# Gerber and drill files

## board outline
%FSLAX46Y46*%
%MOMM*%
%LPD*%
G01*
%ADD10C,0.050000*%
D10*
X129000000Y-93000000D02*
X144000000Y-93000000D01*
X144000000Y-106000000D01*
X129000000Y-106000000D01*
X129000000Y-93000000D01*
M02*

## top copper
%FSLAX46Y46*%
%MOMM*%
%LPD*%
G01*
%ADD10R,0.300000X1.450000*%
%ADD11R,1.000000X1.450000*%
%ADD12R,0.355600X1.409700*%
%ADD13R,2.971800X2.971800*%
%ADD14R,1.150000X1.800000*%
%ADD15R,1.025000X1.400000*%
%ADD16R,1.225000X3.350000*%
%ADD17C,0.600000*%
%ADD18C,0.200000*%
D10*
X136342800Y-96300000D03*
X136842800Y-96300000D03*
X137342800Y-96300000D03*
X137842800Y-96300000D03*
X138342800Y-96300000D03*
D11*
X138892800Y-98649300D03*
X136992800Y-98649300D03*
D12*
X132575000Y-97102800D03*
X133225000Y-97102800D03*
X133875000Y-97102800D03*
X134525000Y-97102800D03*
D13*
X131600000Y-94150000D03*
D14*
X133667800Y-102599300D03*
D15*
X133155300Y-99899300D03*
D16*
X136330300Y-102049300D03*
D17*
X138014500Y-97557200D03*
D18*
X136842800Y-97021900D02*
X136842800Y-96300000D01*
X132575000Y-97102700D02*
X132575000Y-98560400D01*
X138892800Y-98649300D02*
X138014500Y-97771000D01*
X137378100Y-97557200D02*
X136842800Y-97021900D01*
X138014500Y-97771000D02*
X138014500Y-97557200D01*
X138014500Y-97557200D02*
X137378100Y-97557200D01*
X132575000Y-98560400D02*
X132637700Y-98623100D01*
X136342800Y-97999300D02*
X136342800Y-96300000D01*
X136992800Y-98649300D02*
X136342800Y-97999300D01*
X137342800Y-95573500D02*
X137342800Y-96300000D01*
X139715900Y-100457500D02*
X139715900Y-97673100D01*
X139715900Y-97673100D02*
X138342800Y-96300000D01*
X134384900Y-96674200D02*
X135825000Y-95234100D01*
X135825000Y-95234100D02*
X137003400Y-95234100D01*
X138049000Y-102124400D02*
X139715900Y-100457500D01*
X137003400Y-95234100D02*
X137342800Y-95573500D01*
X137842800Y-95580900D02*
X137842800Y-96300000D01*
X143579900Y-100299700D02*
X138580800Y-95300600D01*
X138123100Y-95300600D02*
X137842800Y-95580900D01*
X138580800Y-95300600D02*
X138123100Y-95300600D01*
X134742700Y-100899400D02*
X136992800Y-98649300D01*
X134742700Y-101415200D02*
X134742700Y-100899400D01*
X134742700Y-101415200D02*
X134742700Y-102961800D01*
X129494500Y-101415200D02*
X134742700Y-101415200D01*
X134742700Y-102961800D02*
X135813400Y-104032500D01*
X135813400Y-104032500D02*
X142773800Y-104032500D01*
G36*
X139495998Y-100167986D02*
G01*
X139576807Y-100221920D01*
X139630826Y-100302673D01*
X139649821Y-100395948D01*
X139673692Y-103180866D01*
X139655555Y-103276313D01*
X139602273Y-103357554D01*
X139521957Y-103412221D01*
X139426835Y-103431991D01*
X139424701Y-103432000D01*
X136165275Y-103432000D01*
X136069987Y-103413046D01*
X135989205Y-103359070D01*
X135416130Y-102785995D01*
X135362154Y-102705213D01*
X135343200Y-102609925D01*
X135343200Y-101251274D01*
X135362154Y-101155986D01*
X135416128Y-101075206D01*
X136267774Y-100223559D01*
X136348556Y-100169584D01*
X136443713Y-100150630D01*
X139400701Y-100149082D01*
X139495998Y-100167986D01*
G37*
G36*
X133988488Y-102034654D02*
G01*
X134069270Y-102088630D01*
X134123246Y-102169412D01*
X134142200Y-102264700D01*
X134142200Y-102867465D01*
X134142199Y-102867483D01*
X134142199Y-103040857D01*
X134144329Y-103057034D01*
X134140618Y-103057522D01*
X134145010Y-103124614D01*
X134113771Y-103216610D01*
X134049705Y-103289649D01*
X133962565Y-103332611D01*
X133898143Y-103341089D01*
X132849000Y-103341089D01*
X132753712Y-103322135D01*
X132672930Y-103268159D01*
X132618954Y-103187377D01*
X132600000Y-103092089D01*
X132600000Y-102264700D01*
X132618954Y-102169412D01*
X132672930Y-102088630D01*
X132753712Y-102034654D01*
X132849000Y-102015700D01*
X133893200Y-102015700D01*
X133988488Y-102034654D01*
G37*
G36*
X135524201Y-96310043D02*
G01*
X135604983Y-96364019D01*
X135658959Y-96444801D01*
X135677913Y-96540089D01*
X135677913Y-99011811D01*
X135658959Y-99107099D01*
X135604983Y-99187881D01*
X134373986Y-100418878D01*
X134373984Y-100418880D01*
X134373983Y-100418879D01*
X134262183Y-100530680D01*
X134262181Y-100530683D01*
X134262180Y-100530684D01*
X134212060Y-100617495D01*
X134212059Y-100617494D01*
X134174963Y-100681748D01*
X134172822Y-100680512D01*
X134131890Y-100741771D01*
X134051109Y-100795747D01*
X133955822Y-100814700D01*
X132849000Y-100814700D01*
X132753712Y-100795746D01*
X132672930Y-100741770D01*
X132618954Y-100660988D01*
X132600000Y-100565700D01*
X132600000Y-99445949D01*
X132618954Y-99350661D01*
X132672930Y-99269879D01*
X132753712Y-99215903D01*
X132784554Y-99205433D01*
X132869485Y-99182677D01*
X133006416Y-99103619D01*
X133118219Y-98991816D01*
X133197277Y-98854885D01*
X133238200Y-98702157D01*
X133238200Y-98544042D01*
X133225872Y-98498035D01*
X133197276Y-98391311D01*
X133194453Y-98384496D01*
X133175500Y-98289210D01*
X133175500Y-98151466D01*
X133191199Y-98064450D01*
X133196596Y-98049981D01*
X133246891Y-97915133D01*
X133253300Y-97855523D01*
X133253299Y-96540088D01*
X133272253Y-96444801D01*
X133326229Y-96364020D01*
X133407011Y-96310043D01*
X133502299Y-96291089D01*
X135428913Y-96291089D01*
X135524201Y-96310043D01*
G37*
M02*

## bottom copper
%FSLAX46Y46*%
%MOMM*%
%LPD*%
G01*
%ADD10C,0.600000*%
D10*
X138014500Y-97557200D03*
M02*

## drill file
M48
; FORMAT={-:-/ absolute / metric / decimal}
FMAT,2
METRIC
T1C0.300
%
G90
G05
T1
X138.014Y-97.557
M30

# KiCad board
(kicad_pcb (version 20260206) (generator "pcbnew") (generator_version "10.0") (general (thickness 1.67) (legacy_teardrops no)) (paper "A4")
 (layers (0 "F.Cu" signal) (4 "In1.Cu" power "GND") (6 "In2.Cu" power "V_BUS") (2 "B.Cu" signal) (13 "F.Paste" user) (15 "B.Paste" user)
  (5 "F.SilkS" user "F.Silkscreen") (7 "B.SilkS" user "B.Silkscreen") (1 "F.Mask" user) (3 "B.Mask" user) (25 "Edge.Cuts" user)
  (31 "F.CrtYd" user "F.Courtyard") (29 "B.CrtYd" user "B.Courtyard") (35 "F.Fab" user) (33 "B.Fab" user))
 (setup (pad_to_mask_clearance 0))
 (gr_rect (start 129 93) (end 144 106) (stroke (width 0.05) (type default)) (fill no) (layer "Edge.Cuts"))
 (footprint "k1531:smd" (layer "F.Cu") (at 136.3428 96.3) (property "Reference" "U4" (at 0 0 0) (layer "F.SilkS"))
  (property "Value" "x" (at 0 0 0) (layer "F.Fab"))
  (pad "1" smd rect (at 0 0) (size 0.3 1.45) (layers "F.Cu" "F.Mask") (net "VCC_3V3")))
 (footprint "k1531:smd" (layer "F.Cu") (at 136.8428 96.3) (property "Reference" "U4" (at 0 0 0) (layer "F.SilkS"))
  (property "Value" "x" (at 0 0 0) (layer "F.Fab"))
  (pad "1" smd rect (at 0 0) (size 0.3 1.45) (layers "F.Cu" "F.Mask") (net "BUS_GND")))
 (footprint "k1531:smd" (layer "F.Cu") (at 137.3428 96.3) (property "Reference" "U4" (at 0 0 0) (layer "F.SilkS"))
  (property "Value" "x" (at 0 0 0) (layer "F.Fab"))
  (pad "1" smd rect (at 0 0) (size 0.3 1.45) (layers "F.Cu" "F.Mask") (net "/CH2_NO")))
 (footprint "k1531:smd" (layer "F.Cu") (at 137.8428 96.3) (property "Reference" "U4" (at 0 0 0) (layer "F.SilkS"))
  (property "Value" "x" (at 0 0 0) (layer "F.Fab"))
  (pad "1" smd rect (at 0 0) (size 0.3 1.45) (layers "F.Cu" "F.Mask") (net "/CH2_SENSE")))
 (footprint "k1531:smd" (layer "F.Cu") (at 138.3428 96.3) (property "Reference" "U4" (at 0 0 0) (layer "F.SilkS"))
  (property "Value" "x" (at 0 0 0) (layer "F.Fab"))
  (pad "1" smd rect (at 0 0) (size 0.3 1.45) (layers "F.Cu" "F.Mask") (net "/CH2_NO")))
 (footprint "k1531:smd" (layer "F.Cu") (at 138.8928 98.6493) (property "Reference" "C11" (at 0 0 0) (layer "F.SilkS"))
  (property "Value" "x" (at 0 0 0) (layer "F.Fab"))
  (pad "1" smd rect (at 0 0) (size 1.0 1.45) (layers "F.Cu" "F.Mask") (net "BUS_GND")))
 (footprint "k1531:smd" (layer "F.Cu") (at 136.9928 98.6493) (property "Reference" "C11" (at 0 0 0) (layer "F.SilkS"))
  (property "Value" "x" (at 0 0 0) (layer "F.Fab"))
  (pad "1" smd rect (at 0 0) (size 1.0 1.45) (layers "F.Cu" "F.Mask") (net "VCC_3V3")))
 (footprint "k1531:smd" (layer "F.Cu") (at 132.575 97.1028) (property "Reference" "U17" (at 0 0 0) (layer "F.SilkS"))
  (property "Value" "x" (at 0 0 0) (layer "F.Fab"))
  (pad "1" smd rect (at 0 0) (size 0.3556 1.4097) (layers "F.Cu" "F.Mask") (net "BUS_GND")))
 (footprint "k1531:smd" (layer "F.Cu") (at 133.225 97.1028) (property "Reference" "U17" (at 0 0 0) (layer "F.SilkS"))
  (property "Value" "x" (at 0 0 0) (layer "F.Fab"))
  (pad "1" smd rect (at 0 0) (size 0.3556 1.4097) (layers "F.Cu" "F.Mask") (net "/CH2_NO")))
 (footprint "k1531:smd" (layer "F.Cu") (at 133.875 97.1028) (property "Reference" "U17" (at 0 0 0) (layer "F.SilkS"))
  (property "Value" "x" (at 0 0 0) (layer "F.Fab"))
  (pad "1" smd rect (at 0 0) (size 0.3556 1.4097) (layers "F.Cu" "F.Mask") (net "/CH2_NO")))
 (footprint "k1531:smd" (layer "F.Cu") (at 134.525 97.1028) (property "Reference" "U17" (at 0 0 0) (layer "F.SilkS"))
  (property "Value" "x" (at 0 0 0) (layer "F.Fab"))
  (pad "1" smd rect (at 0 0) (size 0.3556 1.4097) (layers "F.Cu" "F.Mask") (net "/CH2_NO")))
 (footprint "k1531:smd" (layer "F.Cu") (at 131.6 94.15) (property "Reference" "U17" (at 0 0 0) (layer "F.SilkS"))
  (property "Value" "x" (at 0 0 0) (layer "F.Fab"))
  (pad "1" smd rect (at 0 0) (size 2.9718 2.9718) (layers "F.Cu" "F.Mask") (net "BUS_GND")))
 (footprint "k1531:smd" (layer "F.Cu") (at 133.6678 102.5993) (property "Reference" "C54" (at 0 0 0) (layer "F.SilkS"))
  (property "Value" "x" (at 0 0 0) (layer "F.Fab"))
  (pad "1" smd rect (at 0 0) (size 1.15 1.8) (layers "F.Cu" "F.Mask") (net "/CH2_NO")))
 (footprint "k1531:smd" (layer "F.Cu") (at 133.1553 99.8993) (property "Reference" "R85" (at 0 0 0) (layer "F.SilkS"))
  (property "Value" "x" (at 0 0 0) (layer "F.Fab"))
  (pad "1" smd rect (at 0 0) (size 1.025 1.4) (layers "F.Cu" "F.Mask") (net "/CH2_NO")))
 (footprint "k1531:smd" (layer "F.Cu") (at 136.3303 102.0493) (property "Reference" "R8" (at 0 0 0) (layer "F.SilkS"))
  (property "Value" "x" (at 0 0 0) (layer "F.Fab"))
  (pad "1" smd rect (at 0 0) (size 1.225 3.35) (layers "F.Cu" "F.Mask") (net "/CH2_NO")))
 (segment (start 136.8428 97.0219) (end 136.8428 96.3) (width 0.2) (layer "F.Cu") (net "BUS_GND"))
 (segment (start 132.575 97.1027) (end 132.575 98.5604) (width 0.2) (layer "F.Cu") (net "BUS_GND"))
 (segment (start 138.8928 98.6493) (end 138.0145 97.771) (width 0.2) (layer "F.Cu") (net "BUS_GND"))
 (segment (start 137.3781 97.5572) (end 136.8428 97.0219) (width 0.2) (layer "F.Cu") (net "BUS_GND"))
 (segment (start 138.0145 97.771) (end 138.0145 97.5572) (width 0.2) (layer "F.Cu") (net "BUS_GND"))
 (segment (start 138.0145 97.5572) (end 137.3781 97.5572) (width 0.2) (layer "F.Cu") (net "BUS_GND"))
 (segment (start 132.575 98.5604) (end 132.6377 98.6231) (width 0.2) (layer "F.Cu") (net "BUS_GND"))
 (segment (start 136.3428 97.9993) (end 136.3428 96.3) (width 0.2) (layer "F.Cu") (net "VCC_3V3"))
 (segment (start 136.9928 98.6493) (end 136.3428 97.9993) (width 0.2) (layer "F.Cu") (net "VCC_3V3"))
 (segment (start 137.3428 95.5735) (end 137.3428 96.3) (width 0.2) (layer "F.Cu") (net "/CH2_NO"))
 (segment (start 139.7159 100.4575) (end 139.7159 97.6731) (width 0.2) (layer "F.Cu") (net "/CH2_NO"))
 (segment (start 139.7159 97.6731) (end 138.3428 96.3) (width 0.2) (layer "F.Cu") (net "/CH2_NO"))
 (segment (start 134.3849 96.6742) (end 135.825 95.2341) (width 0.2) (layer "F.Cu") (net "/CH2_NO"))
 (segment (start 135.825 95.2341) (end 137.0034 95.2341) (width 0.2) (layer "F.Cu") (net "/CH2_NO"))
 (segment (start 138.049 102.1244) (end 139.7159 100.4575) (width 0.2) (layer "F.Cu") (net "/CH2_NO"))
 (segment (start 137.0034 95.2341) (end 137.3428 95.5735) (width 0.2) (layer "F.Cu") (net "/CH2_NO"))
 (segment (start 137.8428 95.5809) (end 137.8428 96.3) (width 0.2) (layer "F.Cu") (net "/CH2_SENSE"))
 (segment (start 143.5799 100.2997) (end 138.5808 95.3006) (width 0.2) (layer "F.Cu") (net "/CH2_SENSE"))
 (segment (start 138.1231 95.3006) (end 137.8428 95.5809) (width 0.2) (layer "F.Cu") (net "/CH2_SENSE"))
 (segment (start 138.5808 95.3006) (end 138.1231 95.3006) (width 0.2) (layer "F.Cu") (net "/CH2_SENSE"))
 (segment (start 134.7427 100.8994) (end 136.9928 98.6493) (width 0.2) (layer "F.Cu") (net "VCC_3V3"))
 (segment (start 134.7427 101.4152) (end 134.7427 100.8994) (width 0.2) (layer "F.Cu") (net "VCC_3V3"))
 (segment (start 134.7427 101.4152) (end 134.7427 102.9618) (width 0.2) (layer "F.Cu") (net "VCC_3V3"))
 (segment (start 129.4945 101.4152) (end 134.7427 101.4152) (width 0.2) (layer "F.Cu") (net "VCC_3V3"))
 (segment (start 134.7427 102.9618) (end 135.8134 104.0325) (width 0.2) (layer "F.Cu") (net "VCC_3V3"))
 (segment (start 135.8134 104.0325) (end 142.7738 104.0325) (width 0.2) (layer "F.Cu") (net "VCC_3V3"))
 (via (at 138.0145 97.5572) (size 0.6) (drill 0.3) (layers "F.Cu" "B.Cu") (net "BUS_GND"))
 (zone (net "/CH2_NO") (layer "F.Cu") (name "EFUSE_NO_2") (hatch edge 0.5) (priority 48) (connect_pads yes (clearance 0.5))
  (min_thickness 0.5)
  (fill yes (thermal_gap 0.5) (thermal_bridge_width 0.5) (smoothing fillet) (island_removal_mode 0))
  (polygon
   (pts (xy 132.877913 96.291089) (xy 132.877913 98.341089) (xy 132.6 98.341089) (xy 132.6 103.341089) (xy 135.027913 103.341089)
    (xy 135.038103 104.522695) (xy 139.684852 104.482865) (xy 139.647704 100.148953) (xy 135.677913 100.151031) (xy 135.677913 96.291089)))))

